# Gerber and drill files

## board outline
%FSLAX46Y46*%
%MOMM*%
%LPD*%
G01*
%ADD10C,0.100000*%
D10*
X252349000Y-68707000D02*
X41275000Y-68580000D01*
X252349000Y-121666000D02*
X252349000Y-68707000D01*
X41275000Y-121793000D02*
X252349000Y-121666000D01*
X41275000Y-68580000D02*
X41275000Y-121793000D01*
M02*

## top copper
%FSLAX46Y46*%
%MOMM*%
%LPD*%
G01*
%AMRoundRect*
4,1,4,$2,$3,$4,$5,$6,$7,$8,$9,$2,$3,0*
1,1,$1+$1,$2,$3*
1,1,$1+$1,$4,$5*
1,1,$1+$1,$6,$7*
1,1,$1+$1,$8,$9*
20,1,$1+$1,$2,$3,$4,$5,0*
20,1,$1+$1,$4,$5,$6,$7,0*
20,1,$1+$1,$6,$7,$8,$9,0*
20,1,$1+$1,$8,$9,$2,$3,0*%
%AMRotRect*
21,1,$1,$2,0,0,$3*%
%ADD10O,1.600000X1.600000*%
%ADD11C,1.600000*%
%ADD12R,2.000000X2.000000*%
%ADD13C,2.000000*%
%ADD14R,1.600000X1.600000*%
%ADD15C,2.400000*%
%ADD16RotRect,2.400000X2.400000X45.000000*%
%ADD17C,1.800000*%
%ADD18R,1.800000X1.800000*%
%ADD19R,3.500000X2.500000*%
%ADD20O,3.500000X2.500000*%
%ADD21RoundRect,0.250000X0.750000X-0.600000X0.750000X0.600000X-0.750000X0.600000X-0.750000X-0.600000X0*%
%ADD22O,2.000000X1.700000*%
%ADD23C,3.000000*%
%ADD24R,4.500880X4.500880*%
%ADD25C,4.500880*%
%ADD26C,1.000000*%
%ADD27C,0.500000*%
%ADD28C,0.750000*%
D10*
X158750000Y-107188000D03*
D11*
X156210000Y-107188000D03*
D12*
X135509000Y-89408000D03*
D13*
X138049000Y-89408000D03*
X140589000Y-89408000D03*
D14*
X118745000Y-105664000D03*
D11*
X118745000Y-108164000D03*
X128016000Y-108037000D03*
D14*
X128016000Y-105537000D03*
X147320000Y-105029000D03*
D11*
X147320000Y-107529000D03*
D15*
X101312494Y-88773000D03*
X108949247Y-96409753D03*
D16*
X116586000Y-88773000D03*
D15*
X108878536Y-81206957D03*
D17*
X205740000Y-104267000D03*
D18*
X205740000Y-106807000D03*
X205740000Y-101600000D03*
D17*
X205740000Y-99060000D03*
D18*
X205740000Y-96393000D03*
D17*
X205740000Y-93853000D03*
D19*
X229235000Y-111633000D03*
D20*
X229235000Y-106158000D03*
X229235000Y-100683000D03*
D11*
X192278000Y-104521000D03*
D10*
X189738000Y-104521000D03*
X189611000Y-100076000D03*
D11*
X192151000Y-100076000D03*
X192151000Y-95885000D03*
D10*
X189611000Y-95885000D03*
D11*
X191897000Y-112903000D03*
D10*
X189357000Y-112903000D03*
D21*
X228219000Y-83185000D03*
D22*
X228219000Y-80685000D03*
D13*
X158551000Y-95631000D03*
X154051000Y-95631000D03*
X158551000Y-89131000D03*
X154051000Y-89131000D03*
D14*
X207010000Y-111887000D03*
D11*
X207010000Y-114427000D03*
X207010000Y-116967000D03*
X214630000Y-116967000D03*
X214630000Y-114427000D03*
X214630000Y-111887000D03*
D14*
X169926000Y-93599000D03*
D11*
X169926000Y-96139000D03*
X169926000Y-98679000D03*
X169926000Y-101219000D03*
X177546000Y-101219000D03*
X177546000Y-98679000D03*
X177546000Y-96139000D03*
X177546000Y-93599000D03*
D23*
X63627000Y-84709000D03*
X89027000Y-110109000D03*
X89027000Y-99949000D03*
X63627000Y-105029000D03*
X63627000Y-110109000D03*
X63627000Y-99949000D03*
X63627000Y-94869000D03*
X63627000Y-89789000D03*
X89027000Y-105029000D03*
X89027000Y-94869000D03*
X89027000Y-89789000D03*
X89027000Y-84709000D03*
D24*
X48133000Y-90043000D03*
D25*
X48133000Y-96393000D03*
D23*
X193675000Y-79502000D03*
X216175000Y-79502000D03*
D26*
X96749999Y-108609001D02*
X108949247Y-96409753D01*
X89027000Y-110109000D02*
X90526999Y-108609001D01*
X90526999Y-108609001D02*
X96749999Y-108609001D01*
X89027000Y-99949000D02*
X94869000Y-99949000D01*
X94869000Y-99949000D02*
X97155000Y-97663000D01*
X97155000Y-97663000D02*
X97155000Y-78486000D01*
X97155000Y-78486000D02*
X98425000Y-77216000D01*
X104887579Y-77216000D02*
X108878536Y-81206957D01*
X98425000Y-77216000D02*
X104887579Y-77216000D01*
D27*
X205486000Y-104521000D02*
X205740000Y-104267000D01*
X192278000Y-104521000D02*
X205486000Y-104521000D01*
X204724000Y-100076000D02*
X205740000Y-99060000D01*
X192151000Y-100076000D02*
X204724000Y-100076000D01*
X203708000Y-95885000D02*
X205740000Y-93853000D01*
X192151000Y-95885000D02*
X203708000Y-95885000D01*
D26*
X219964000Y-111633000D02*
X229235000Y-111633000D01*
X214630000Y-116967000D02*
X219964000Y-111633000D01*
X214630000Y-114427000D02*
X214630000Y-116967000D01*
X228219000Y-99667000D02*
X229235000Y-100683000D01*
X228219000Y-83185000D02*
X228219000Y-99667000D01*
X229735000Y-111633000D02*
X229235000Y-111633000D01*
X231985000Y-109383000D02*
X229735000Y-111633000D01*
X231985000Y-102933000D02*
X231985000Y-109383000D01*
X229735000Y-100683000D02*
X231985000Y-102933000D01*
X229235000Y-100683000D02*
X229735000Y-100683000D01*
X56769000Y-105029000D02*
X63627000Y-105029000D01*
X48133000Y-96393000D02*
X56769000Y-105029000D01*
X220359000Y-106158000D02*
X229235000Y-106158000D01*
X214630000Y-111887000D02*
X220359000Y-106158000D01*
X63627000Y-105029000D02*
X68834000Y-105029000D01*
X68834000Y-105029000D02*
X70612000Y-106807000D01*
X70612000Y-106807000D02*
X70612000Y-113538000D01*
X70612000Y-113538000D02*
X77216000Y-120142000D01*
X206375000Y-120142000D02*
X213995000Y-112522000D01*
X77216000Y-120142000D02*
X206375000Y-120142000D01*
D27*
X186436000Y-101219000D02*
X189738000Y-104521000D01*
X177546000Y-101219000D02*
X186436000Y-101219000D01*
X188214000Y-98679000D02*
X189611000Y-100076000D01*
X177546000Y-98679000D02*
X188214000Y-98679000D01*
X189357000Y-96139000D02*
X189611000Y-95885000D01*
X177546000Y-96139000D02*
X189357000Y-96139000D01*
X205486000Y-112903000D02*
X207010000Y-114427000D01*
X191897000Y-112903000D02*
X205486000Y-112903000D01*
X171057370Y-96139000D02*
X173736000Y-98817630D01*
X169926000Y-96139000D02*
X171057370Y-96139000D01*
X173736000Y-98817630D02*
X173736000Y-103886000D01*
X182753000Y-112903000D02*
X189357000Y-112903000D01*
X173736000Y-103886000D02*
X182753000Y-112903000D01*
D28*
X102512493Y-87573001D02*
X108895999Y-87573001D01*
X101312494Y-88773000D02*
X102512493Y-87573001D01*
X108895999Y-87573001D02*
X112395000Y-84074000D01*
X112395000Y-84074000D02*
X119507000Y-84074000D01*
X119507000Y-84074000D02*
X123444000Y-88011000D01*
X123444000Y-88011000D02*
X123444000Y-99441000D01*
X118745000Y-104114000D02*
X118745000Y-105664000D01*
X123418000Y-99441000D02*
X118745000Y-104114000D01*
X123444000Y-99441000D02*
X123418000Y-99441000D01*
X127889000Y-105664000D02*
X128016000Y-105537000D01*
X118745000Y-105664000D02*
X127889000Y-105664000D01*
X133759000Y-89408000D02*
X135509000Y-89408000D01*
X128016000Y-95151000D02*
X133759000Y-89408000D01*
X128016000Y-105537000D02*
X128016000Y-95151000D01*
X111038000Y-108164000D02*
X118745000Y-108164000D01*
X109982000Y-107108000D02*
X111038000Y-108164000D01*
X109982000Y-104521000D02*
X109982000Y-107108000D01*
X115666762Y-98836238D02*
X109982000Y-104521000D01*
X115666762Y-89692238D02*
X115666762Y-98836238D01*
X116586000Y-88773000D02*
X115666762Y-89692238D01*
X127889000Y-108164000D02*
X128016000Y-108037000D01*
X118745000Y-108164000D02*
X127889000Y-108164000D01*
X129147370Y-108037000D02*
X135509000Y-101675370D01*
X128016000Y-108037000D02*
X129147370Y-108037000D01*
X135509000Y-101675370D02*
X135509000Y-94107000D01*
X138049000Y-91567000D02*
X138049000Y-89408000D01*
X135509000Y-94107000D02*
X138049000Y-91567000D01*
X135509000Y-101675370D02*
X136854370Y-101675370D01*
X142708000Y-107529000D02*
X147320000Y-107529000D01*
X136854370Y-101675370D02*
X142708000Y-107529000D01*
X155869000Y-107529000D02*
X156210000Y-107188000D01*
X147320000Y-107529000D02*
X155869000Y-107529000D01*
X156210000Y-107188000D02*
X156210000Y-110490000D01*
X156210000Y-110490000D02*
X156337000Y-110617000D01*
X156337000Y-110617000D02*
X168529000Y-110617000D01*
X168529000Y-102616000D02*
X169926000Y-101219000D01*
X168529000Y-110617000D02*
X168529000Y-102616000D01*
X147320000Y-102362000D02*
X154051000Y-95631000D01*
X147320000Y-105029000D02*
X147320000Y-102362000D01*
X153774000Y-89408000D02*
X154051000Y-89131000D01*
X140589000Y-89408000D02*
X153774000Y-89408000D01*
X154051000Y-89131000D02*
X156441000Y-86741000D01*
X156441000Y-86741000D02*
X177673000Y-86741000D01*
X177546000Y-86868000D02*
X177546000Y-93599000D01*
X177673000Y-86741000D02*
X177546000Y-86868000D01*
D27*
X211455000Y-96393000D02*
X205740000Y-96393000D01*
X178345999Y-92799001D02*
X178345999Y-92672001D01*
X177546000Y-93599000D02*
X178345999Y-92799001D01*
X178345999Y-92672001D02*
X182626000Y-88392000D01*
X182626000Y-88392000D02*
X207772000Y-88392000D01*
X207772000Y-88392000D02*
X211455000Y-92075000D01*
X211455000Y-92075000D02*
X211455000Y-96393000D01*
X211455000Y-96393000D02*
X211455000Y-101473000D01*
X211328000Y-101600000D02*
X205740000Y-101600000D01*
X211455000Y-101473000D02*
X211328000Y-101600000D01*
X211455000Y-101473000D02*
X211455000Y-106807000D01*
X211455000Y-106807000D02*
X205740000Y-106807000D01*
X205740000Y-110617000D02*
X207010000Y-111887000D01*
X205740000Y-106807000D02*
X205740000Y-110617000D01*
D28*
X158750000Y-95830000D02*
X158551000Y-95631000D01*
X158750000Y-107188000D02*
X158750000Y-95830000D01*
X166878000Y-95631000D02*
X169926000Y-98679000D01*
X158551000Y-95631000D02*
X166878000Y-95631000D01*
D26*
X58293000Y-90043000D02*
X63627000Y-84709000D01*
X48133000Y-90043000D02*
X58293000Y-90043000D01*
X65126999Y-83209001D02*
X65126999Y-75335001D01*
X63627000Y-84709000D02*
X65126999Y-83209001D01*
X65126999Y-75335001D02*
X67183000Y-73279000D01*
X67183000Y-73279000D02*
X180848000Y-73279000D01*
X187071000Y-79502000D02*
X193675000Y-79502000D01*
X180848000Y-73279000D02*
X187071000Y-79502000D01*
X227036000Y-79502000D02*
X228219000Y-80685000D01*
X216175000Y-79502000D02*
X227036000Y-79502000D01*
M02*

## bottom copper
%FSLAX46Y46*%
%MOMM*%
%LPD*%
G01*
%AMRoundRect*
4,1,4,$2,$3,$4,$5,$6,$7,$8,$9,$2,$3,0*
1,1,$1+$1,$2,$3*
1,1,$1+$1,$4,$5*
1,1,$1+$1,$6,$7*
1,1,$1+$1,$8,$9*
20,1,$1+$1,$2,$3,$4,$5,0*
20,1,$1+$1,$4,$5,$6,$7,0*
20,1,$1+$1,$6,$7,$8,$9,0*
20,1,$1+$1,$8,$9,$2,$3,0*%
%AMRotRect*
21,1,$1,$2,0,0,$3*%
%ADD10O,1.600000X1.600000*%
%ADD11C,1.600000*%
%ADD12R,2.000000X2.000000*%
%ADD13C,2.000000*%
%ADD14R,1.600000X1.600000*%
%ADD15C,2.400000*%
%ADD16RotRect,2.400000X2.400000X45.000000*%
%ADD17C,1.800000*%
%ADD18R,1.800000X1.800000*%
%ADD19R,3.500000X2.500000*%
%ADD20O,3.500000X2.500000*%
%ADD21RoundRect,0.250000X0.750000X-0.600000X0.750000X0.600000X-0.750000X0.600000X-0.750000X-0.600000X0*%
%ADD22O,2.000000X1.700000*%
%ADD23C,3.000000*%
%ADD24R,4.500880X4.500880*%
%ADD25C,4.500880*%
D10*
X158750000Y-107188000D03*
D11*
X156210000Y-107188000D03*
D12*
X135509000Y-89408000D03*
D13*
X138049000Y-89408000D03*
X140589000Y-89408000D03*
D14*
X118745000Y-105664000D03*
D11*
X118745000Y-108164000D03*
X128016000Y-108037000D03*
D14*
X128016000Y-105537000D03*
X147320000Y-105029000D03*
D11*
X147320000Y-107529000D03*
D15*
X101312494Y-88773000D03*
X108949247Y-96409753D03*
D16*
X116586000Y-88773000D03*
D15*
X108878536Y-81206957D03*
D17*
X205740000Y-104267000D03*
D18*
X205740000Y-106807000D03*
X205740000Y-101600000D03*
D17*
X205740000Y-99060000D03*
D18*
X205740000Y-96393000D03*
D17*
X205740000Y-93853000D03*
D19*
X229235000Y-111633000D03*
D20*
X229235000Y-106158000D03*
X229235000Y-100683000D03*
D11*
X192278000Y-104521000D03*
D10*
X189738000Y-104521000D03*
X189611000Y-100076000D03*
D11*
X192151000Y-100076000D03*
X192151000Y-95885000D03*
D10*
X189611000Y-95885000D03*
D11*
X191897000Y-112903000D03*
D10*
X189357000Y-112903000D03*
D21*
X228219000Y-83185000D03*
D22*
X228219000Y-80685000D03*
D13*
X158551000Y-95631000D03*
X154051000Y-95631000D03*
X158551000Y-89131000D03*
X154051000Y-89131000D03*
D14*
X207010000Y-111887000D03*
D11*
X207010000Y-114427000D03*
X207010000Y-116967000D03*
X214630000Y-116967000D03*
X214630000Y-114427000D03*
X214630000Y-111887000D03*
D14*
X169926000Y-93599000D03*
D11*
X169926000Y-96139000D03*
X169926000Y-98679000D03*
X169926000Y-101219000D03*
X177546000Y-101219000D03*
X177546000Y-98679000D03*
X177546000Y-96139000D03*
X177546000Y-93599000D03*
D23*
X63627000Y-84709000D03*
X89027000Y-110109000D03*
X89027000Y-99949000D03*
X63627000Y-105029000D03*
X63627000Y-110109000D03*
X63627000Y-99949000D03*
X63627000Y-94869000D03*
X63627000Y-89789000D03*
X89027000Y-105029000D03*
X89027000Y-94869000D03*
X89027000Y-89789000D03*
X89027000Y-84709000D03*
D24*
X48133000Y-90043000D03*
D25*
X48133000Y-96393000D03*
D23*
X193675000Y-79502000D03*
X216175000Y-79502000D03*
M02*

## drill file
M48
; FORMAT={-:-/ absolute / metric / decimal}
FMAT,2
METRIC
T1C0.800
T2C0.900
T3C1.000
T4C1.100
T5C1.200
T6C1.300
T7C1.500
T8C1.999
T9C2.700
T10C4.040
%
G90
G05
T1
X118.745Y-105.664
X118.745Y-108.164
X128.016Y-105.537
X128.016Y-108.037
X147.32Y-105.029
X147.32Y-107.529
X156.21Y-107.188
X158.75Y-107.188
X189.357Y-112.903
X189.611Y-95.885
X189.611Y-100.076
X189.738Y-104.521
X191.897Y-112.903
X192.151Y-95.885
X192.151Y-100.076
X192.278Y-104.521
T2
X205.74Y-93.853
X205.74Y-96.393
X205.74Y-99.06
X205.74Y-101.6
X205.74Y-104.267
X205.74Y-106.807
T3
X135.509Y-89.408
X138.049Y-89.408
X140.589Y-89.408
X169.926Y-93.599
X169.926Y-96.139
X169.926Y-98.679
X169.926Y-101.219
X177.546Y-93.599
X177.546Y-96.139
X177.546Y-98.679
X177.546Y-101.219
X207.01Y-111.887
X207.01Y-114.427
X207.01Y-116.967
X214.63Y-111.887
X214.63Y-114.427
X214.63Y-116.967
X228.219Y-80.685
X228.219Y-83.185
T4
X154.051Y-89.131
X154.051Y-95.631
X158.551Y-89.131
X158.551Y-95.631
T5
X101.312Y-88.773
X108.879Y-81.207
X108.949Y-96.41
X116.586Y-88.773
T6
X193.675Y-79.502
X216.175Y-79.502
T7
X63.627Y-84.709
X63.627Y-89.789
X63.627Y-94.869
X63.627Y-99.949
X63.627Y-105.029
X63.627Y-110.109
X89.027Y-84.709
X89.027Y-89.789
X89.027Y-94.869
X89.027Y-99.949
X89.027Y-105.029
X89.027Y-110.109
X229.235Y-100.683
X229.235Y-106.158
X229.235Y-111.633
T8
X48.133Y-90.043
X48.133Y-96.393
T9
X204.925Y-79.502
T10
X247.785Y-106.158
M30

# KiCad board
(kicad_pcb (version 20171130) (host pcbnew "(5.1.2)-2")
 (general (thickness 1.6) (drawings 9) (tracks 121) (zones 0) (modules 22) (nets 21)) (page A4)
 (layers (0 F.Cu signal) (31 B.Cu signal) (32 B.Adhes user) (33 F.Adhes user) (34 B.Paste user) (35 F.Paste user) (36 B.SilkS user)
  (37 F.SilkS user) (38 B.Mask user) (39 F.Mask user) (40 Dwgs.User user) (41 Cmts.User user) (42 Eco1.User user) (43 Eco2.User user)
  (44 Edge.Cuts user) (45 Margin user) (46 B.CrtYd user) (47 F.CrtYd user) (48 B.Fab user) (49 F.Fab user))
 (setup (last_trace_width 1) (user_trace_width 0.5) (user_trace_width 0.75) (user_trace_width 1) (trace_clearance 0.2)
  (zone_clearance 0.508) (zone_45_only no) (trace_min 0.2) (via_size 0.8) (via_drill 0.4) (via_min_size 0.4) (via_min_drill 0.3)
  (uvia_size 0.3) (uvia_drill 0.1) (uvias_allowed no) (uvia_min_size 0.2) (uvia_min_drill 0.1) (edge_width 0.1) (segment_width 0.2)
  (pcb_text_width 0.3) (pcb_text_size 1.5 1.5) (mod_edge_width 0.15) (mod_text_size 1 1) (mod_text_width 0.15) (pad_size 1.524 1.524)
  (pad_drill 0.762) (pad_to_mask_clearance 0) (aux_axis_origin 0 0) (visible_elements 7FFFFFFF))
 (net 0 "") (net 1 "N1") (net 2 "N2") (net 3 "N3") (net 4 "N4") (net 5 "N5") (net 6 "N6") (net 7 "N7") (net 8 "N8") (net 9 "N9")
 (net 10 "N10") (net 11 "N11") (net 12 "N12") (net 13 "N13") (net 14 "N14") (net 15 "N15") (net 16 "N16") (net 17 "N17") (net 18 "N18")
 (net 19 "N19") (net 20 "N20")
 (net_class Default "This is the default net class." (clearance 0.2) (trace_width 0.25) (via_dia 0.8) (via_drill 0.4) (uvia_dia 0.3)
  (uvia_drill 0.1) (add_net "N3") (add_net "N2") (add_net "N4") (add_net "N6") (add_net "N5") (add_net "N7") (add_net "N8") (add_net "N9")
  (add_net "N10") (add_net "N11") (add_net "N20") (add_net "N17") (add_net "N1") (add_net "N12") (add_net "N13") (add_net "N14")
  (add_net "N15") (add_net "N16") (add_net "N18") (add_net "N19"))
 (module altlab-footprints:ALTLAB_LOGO (layer F.Cu) (at 136.271 78.867)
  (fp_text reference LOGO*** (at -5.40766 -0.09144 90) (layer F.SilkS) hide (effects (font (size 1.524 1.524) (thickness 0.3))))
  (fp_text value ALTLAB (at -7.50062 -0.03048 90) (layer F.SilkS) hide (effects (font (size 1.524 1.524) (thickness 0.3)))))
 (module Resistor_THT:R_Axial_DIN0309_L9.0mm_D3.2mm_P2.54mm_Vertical (layer F.Cu) (at 156.21 107.188)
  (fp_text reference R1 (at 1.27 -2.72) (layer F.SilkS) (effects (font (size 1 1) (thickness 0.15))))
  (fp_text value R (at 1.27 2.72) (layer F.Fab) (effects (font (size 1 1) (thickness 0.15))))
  (pad 2 thru_hole oval (at 2.54 0) (size 1.6 1.6) (drill 0.8) (layers *.Cu *.Mask) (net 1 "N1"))
  (pad 1 thru_hole circle (at 0 0) (size 1.6 1.6) (drill 0.8) (layers *.Cu *.Mask) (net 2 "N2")))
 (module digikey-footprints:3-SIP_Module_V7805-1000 (layer F.Cu) (at 135.509 89.408)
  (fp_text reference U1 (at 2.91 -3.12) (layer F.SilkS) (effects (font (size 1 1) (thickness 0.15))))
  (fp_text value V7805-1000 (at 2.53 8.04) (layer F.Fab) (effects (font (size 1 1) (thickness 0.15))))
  (pad 1 thru_hole rect (at 0 0) (size 2 2) (drill 1) (layers *.Cu *.Mask) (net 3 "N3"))
  (pad 2 thru_hole circle (at 2.54 0) (size 2 2) (drill 1) (layers *.Cu *.Mask) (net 2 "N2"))
  (pad 3 thru_hole circle (at 5.08 0) (size 2 2) (drill 1) (layers *.Cu *.Mask) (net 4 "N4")))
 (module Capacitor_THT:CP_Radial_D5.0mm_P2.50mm (layer F.Cu) (at 118.745 105.664 270)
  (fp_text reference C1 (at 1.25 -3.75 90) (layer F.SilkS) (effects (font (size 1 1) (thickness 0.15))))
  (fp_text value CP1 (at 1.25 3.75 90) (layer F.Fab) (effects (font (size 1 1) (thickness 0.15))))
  (pad 1 thru_hole rect (at 0 0 270) (size 1.6 1.6) (drill 0.8) (layers *.Cu *.Mask) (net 3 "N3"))
  (pad 2 thru_hole circle (at 2.5 0 270) (size 1.6 1.6) (drill 0.8) (layers *.Cu *.Mask) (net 2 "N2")))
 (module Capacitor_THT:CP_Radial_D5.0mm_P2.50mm (layer F.Cu) (at 128.016 105.537 270)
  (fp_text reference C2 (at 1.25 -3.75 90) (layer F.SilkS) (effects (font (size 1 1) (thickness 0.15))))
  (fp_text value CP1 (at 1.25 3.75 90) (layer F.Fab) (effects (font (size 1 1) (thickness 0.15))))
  (pad 2 thru_hole circle (at 2.5 0 270) (size 1.6 1.6) (drill 0.8) (layers *.Cu *.Mask) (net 2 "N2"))
  (pad 1 thru_hole rect (at 0 0 270) (size 1.6 1.6) (drill 0.8) (layers *.Cu *.Mask) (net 3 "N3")))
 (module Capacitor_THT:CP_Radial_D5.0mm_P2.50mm (layer F.Cu) (at 147.32 105.029 270)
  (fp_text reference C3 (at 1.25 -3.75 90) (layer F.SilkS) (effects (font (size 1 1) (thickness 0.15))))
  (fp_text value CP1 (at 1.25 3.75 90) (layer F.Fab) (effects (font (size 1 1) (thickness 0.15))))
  (pad 1 thru_hole rect (at 0 0 270) (size 1.6 1.6) (drill 0.8) (layers *.Cu *.Mask) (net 4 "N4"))
  (pad 2 thru_hole circle (at 2.5 0 270) (size 1.6 1.6) (drill 0.8) (layers *.Cu *.Mask) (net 2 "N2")))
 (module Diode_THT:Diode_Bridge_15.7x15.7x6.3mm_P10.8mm (layer F.Cu) (at 116.586 88.773 225)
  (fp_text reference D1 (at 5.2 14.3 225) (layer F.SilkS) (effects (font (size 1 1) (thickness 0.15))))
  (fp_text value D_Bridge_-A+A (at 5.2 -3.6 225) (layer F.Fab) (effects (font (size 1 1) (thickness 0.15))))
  (pad 3 thru_hole circle (at 10.8 10.8 45) (size 2.4 2.4) (drill 1.2) (layers *.Cu *.Mask) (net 3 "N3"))
  (pad 4 thru_hole circle (at 10.8 0 45) (size 2.4 2.4) (drill 1.2) (layers *.Cu *.Mask) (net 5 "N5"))
  (pad 1 thru_hole rect (at 0 0 45) (size 2.4 2.4) (drill 1.2) (layers *.Cu *.Mask) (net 2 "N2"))
  (pad 2 thru_hole circle (at 0.1 10.8 45) (size 2.4 2.4) (drill 1.2) (layers *.Cu *.Mask) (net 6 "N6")))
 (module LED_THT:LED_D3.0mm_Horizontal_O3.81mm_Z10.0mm (layer F.Cu) (at 205.74 106.807 90)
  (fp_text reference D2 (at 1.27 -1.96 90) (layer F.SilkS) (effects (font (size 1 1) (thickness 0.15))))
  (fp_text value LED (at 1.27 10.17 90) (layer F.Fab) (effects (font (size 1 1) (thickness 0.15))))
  (pad 2 thru_hole circle (at 2.54 0 90) (size 1.8 1.8) (drill 0.9) (layers *.Cu *.Mask) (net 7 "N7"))
  (pad 1 thru_hole rect (at 0 0 90) (size 1.8 1.8) (drill 0.9) (layers *.Cu *.Mask) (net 4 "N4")))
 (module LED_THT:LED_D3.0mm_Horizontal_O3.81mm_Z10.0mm (layer F.Cu) (at 205.74 101.6 90)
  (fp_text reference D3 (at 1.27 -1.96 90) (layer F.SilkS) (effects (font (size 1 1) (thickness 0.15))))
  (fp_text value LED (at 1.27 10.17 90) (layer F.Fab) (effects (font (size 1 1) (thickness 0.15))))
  (pad 1 thru_hole rect (at 0 0 90) (size 1.8 1.8) (drill 0.9) (layers *.Cu *.Mask) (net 4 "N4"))
  (pad 2 thru_hole circle (at 2.54 0 90) (size 1.8 1.8) (drill 0.9) (layers *.Cu *.Mask) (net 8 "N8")))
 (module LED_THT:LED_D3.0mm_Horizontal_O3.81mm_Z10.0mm (layer F.Cu) (at 205.74 96.393 90)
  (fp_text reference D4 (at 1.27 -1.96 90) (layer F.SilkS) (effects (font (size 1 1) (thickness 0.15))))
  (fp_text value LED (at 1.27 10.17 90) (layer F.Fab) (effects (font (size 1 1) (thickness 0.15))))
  (pad 1 thru_hole rect (at 0 0 90) (size 1.8 1.8) (drill 0.9) (layers *.Cu *.Mask) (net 4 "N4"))
  (pad 2 thru_hole circle (at 2.54 0 90) (size 1.8 1.8) (drill 0.9) (layers *.Cu *.Mask) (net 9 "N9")))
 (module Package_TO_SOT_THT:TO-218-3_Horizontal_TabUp (layer F.Cu) (at 229.235 111.633 90)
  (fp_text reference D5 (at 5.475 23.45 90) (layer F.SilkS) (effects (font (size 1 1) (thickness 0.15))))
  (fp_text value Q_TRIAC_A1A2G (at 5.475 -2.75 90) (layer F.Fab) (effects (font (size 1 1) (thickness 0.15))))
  (pad "" np_thru_hole oval (at 5.475 18.55 90) (size 4.04 4.04) (drill 4.04) (layers *.Cu *.Mask))
  (pad 1 thru_hole rect (at 0 0 90) (size 2.5 3.5) (drill 1.5) (layers *.Cu *.Mask) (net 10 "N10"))
  (pad 2 thru_hole oval (at 5.475 0 90) (size 2.5 3.5) (drill 1.5) (layers *.Cu *.Mask) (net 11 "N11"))
  (pad 3 thru_hole oval (at 10.95 0 90) (size 2.5 3.5) (drill 1.5) (layers *.Cu *.Mask) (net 10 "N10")))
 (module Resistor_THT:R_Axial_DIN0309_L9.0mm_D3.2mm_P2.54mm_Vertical (layer F.Cu) (at 192.278 104.521 180)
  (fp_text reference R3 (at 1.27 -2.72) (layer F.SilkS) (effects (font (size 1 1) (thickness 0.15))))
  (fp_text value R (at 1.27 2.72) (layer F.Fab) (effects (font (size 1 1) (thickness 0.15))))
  (pad 1 thru_hole circle (at 0 0 180) (size 1.6 1.6) (drill 0.8) (layers *.Cu *.Mask) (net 7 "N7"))
  (pad 2 thru_hole oval (at 2.54 0 180) (size 1.6 1.6) (drill 0.8) (layers *.Cu *.Mask) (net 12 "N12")))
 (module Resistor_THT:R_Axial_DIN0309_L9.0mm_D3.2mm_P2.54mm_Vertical (layer F.Cu) (at 192.151 100.076 180)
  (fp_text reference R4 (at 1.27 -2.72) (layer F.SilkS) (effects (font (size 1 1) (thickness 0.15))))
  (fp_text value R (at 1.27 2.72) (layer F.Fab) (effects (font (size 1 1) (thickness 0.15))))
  (pad 2 thru_hole oval (at 2.54 0 180) (size 1.6 1.6) (drill 0.8) (layers *.Cu *.Mask) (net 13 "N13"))
  (pad 1 thru_hole circle (at 0 0 180) (size 1.6 1.6) (drill 0.8) (layers *.Cu *.Mask) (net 8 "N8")))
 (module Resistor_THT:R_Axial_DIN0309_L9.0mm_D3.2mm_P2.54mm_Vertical (layer F.Cu) (at 192.151 95.885 180)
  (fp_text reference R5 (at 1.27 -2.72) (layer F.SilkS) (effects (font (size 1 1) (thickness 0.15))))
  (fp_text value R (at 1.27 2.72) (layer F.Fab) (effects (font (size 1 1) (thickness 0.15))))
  (pad 1 thru_hole circle (at 0 0 180) (size 1.6 1.6) (drill 0.8) (layers *.Cu *.Mask) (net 9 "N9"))
  (pad 2 thru_hole oval (at 2.54 0 180) (size 1.6 1.6) (drill 0.8) (layers *.Cu *.Mask) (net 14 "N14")))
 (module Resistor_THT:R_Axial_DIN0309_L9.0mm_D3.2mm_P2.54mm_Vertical (layer F.Cu) (at 191.897 112.903 180)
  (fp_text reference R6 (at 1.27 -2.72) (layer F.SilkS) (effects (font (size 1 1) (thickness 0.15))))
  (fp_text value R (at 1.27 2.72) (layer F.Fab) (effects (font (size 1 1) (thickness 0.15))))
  (pad 1 thru_hole circle (at 0 0 180) (size 1.6 1.6) (drill 0.8) (layers *.Cu *.Mask) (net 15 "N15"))
  (pad 2 thru_hole oval (at 2.54 0 180) (size 1.6 1.6) (drill 0.8) (layers *.Cu *.Mask) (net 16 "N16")))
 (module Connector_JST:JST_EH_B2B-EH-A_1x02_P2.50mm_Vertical (layer F.Cu) (at 228.219 83.185 90)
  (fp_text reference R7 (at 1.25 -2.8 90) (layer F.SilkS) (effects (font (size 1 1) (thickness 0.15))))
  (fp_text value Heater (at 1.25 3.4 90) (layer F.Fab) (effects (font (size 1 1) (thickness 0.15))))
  (pad 1 thru_hole roundrect (at 0 0 90) (size 1.7 2) (drill 1) (layers *.Cu *.Mask) (roundrect_rratio 0.147059) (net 10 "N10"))
  (pad 2 thru_hole oval (at 2.5 0 90) (size 1.7 2) (drill 1) (layers *.Cu *.Mask) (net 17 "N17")))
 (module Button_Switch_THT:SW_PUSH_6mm (layer F.Cu) (at 154.051 95.631 90)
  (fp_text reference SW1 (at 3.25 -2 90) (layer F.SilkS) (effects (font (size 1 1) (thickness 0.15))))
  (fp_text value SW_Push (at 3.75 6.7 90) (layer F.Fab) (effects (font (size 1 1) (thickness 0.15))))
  (pad 2 thru_hole circle (at 0 4.5 180) (size 2 2) (drill 1.1) (layers *.Cu *.Mask) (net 1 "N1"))
  (pad 1 thru_hole circle (at 0 0 180) (size 2 2) (drill 1.1) (layers *.Cu *.Mask) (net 4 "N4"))
  (pad 2 thru_hole circle (at 6.5 4.5 180) (size 2 2) (drill 1.1) (layers *.Cu *.Mask) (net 1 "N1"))
  (pad 1 thru_hole circle (at 6.5 0 180) (size 2 2) (drill 1.1) (layers *.Cu *.Mask) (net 4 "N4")))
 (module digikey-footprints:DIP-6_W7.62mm (layer F.Cu) (at 207.01 111.887)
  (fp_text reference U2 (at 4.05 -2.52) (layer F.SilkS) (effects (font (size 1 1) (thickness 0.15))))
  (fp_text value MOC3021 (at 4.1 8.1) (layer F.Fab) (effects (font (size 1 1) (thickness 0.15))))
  (pad 1 thru_hole rect (at 0 0) (size 1.6 1.6) (drill 1) (layers *.Cu *.Mask) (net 4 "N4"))
  (pad 2 thru_hole circle (at 0 2.54) (size 1.6 1.6) (drill 1) (layers *.Cu *.Mask) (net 15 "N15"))
  (pad 3 thru_hole circle (at 0 5.08) (size 1.6 1.6) (drill 1) (layers *.Cu *.Mask) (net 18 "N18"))
  (pad 4 thru_hole circle (at 7.62 5.08) (size 1.6 1.6) (drill 1) (layers *.Cu *.Mask) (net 10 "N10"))
  (pad 5 thru_hole circle (at 7.62 2.54) (size 1.6 1.6) (drill 1) (layers *.Cu *.Mask) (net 10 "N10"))
  (pad 6 thru_hole circle (at 7.62 0) (size 1.6 1.6) (drill 1) (layers *.Cu *.Mask) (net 11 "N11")))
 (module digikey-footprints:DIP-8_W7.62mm (layer F.Cu) (at 169.926 93.599)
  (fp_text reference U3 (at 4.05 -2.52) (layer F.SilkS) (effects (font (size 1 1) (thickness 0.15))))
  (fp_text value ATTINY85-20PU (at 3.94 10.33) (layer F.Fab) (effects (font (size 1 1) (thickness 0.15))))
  (pad 1 thru_hole rect (at 0 0) (size 1.6 1.6) (drill 1) (layers *.Cu *.Mask) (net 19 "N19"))
  (pad 2 thru_hole circle (at 0 2.54) (size 1.6 1.6) (drill 1) (layers *.Cu *.Mask) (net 16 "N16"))
  (pad 3 thru_hole circle (at 0 5.08) (size 1.6 1.6) (drill 1) (layers *.Cu *.Mask) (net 1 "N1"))
  (pad 4 thru_hole circle (at 0 7.62) (size 1.6 1.6) (drill 1) (layers *.Cu *.Mask) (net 2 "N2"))
  (pad 5 thru_hole circle (at 7.62 7.62) (size 1.6 1.6) (drill 1) (layers *.Cu *.Mask) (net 12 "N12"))
  (pad 6 thru_hole circle (at 7.62 5.08) (size 1.6 1.6) (drill 1) (layers *.Cu *.Mask) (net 13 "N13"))
  (pad 7 thru_hole circle (at 7.62 2.54) (size 1.6 1.6) (drill 1) (layers *.Cu *.Mask) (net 14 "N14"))
  (pad 8 thru_hole circle (at 7.62 0) (size 1.6 1.6) (drill 1) (layers *.Cu *.Mask) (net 4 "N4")))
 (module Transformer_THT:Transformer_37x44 (layer F.Cu) (at 63.627 105.029 90)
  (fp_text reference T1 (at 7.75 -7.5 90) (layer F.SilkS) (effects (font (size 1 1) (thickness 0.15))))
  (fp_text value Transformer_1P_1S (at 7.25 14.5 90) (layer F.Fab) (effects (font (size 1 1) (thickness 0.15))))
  (pad 2 thru_hole circle (at 20.32 0 90) (size 3 3) (drill 1.5) (layers *.Cu *.Mask) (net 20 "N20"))
  (pad 4 thru_hole circle (at -5.08 25.4 90) (size 3 3) (drill 1.5) (layers *.Cu *.Mask) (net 5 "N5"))
  (pad 3 thru_hole circle (at 5.08 25.4 90) (size 3 3) (drill 1.5) (layers *.Cu *.Mask) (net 6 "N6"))
  (pad 1 thru_hole circle (at 0 0 90) (size 3 3) (drill 1.5) (layers *.Cu *.Mask) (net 11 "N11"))
  (pad "" thru_hole circle (at -5.08 0 90) (size 3 3) (drill 1.5) (layers *.Cu *.Mask))
  (pad "" thru_hole circle (at 5.08 0 90) (size 3 3) (drill 1.5) (layers *.Cu *.Mask))
  (pad "" thru_hole circle (at 10.16 0 90) (size 3 3) (drill 1.5) (layers *.Cu *.Mask))
  (pad "" thru_hole circle (at 15.24 0 90) (size 3 3) (drill 1.5) (layers *.Cu *.Mask))
  (pad "" thru_hole circle (at 0 25.4 90) (size 3 3) (drill 1.5) (layers *.Cu *.Mask))
  (pad "" thru_hole circle (at 10.16 25.4 90) (size 3 3) (drill 1.5) (layers *.Cu *.Mask))
  (pad "" thru_hole circle (at 15.24 25.4 90) (size 3 3) (drill 1.5) (layers *.Cu *.Mask))
  (pad "" thru_hole circle (at 20.32 25.4 90) (size 3 3) (drill 1.5) (layers *.Cu *.Mask)))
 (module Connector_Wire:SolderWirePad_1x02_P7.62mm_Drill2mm (layer F.Cu) (at 48.133 90.043 270)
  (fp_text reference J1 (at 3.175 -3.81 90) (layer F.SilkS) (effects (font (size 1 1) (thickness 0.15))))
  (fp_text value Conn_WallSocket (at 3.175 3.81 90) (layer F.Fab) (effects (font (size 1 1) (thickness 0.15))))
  (pad 1 thru_hole rect (at 0 0 270) (size 4.50088 4.50088) (drill 1.99898) (layers *.Cu *.Mask) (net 20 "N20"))
  (pad 2 thru_hole circle (at 6.35 0 270) (size 4.50088 4.50088) (drill 1.99898) (layers *.Cu *.Mask) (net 11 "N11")))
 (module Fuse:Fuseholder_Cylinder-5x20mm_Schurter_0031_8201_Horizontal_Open (layer F.Cu) (at 193.675 79.502)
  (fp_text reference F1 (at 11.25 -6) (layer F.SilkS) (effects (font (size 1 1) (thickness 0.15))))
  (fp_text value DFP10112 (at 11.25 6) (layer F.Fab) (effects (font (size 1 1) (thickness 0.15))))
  (pad 1 thru_hole circle (at 0 0) (size 3 3) (drill 1.3) (layers *.Cu *.Mask) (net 20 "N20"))
  (pad 2 thru_hole circle (at 22.5 0) (size 3 3) (drill 1.3) (layers *.Cu *.Mask) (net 17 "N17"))
  (pad "" np_thru_hole circle (at 11.25 0) (size 2.7 2.7) (drill 2.7) (layers *.Cu *.Mask)))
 (gr_line (start 252.349 68.707) (end 41.275 68.58) (layer Edge.Cuts) (width 0.1))
 (gr_line (start 252.349 121.666) (end 252.349 68.707) (layer Edge.Cuts) (width 0.1))
 (gr_line (start 41.275 121.793) (end 252.349 121.666) (layer Edge.Cuts) (width 0.1))
 (gr_line (start 41.275 68.58) (end 41.275 121.793) (layer Edge.Cuts) (width 0.1))
 (segment (start 96.749999 108.609001) (end 108.949247 96.409753) (width 1) (layer F.Cu) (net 5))
 (segment (start 89.027 110.109) (end 90.526999 108.609001) (width 1) (layer F.Cu) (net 5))
 (segment (start 90.526999 108.609001) (end 96.749999 108.609001) (width 1) (layer F.Cu) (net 5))
 (segment (start 89.027 99.949) (end 94.869 99.949) (width 1) (layer F.Cu) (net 6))
 (segment (start 94.869 99.949) (end 97.155 97.663) (width 1) (layer F.Cu) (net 6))
 (segment (start 97.155 97.663) (end 97.155 78.486) (width 1) (layer F.Cu) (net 6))
 (segment (start 97.155 78.486) (end 98.425 77.216) (width 1) (layer F.Cu) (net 6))
 (segment (start 104.887579 77.216) (end 108.878536 81.206957) (width 1) (layer F.Cu) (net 6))
 (segment (start 98.425 77.216) (end 104.887579 77.216) (width 1) (layer F.Cu) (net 6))
 (segment (start 205.486 104.521) (end 205.74 104.267) (width 0.5) (layer F.Cu) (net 7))
 (segment (start 192.278 104.521) (end 205.486 104.521) (width 0.5) (layer F.Cu) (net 7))
 (segment (start 204.724 100.076) (end 205.74 99.06) (width 0.5) (layer F.Cu) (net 8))
 (segment (start 192.151 100.076) (end 204.724 100.076) (width 0.5) (layer F.Cu) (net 8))
 (segment (start 203.708 95.885) (end 205.74 93.853) (width 0.5) (layer F.Cu) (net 9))
 (segment (start 192.151 95.885) (end 203.708 95.885) (width 0.5) (layer F.Cu) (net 9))
 (segment (start 219.964 111.633) (end 229.235 111.633) (width 1) (layer F.Cu) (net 10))
 (segment (start 214.63 116.967) (end 219.964 111.633) (width 1) (layer F.Cu) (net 10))
 (segment (start 214.63 114.427) (end 214.63 116.967) (width 1) (layer F.Cu) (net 10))
 (segment (start 228.219 99.667) (end 229.235 100.683) (width 1) (layer F.Cu) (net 10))
 (segment (start 228.219 83.185) (end 228.219 99.667) (width 1) (layer F.Cu) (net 10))
 (segment (start 229.735 111.633) (end 229.235 111.633) (width 1) (layer F.Cu) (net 10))
 (segment (start 231.985 109.383) (end 229.735 111.633) (width 1) (layer F.Cu) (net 10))
 (segment (start 231.985 102.933) (end 231.985 109.383) (width 1) (layer F.Cu) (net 10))
 (segment (start 229.735 100.683) (end 231.985 102.933) (width 1) (layer F.Cu) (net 10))
 (segment (start 229.235 100.683) (end 229.735 100.683) (width 1) (layer F.Cu) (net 10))
 (segment (start 56.769 105.029) (end 63.627 105.029) (width 1) (layer F.Cu) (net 11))
 (segment (start 48.133 96.393) (end 56.769 105.029) (width 1) (layer F.Cu) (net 11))
 (segment (start 220.359 106.158) (end 229.235 106.158) (width 1) (layer F.Cu) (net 11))
 (segment (start 214.63 111.887) (end 220.359 106.158) (width 1) (layer F.Cu) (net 11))
 (segment (start 63.627 105.029) (end 68.834 105.029) (width 1) (layer F.Cu) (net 11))
 (segment (start 68.834 105.029) (end 70.612 106.807) (width 1) (layer F.Cu) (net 11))
 (segment (start 70.612 106.807) (end 70.612 113.538) (width 1) (layer F.Cu) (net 11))
 (segment (start 70.612 113.538) (end 77.216 120.142) (width 1) (layer F.Cu) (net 11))
 (segment (start 206.375 120.142) (end 213.995 112.522) (width 1) (layer F.Cu) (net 11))
 (segment (start 77.216 120.142) (end 206.375 120.142) (width 1) (layer F.Cu) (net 11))
 (segment (start 186.436 101.219) (end 189.738 104.521) (width 0.5) (layer F.Cu) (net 12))
 (segment (start 177.546 101.219) (end 186.436 101.219) (width 0.5) (layer F.Cu) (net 12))
 (segment (start 188.214 98.679) (end 189.611 100.076) (width 0.5) (layer F.Cu) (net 13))
 (segment (start 177.546 98.679) (end 188.214 98.679) (width 0.5) (layer F.Cu) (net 13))
 (segment (start 189.357 96.139) (end 189.611 95.885) (width 0.5) (layer F.Cu) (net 14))
 (segment (start 177.546 96.139) (end 189.357 96.139) (width 0.5) (layer F.Cu) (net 14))
 (segment (start 205.486 112.903) (end 207.01 114.427) (width 0.5) (layer F.Cu) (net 15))
 (segment (start 191.897 112.903) (end 205.486 112.903) (width 0.5) (layer F.Cu) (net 15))
 (segment (start 171.05737 96.139) (end 173.736 98.81763) (width 0.5) (layer F.Cu) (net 16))
 (segment (start 169.926 96.139) (end 171.05737 96.139) (width 0.5) (layer F.Cu) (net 16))
 (segment (start 173.736 98.81763) (end 173.736 103.886) (width 0.5) (layer F.Cu) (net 16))
 (segment (start 182.753 112.903) (end 189.357 112.903) (width 0.5) (layer F.Cu) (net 16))
 (segment (start 173.736 103.886) (end 182.753 112.903) (width 0.5) (layer F.Cu) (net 16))
 (segment (start 102.512493 87.573001) (end 108.895999 87.573001) (width 0.75) (layer F.Cu) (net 3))
 (segment (start 101.312494 88.773) (end 102.512493 87.573001) (width 0.75) (layer F.Cu) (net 3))
 (segment (start 108.895999 87.573001) (end 112.395 84.074) (width 0.75) (layer F.Cu) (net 3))
 (segment (start 112.395 84.074) (end 119.507 84.074) (width 0.75) (layer F.Cu) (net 3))
 (segment (start 119.507 84.074) (end 123.444 88.011) (width 0.75) (layer F.Cu) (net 3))
 (segment (start 123.444 88.011) (end 123.444 99.441) (width 0.75) (layer F.Cu) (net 3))
 (segment (start 118.745 104.114) (end 118.745 105.664) (width 0.75) (layer F.Cu) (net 3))
 (segment (start 123.418 99.441) (end 118.745 104.114) (width 0.75) (layer F.Cu) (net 3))
 (segment (start 123.444 99.441) (end 123.418 99.441) (width 0.75) (layer F.Cu) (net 3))
 (segment (start 127.889 105.664) (end 128.016 105.537) (width 0.75) (layer F.Cu) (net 3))
 (segment (start 118.745 105.664) (end 127.889 105.664) (width 0.75) (layer F.Cu) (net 3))
 (segment (start 133.759 89.408) (end 135.509 89.408) (width 0.75) (layer F.Cu) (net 3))
 (segment (start 128.016 95.151) (end 133.759 89.408) (width 0.75) (layer F.Cu) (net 3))
 (segment (start 128.016 105.537) (end 128.016 95.151) (width 0.75) (layer F.Cu) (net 3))
 (segment (start 111.038 108.164) (end 118.745 108.164) (width 0.75) (layer F.Cu) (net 2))
 (segment (start 109.982 107.108) (end 111.038 108.164) (width 0.75) (layer F.Cu) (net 2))
 (segment (start 109.982 104.521) (end 109.982 107.108) (width 0.75) (layer F.Cu) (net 2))
 (segment (start 115.666762 98.836238) (end 109.982 104.521) (width 0.75) (layer F.Cu) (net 2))
 (segment (start 115.666762 89.692238) (end 115.666762 98.836238) (width 0.75) (layer F.Cu) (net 2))
 (segment (start 116.586 88.773) (end 115.666762 89.692238) (width 0.75) (layer F.Cu) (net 2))
 (segment (start 127.889 108.164) (end 128.016 108.037) (width 0.75) (layer F.Cu) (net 2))
 (segment (start 118.745 108.164) (end 127.889 108.164) (width 0.75) (layer F.Cu) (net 2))
 (segment (start 129.14737 108.037) (end 135.509 101.67537) (width 0.75) (layer F.Cu) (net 2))
 (segment (start 128.016 108.037) (end 129.14737 108.037) (width 0.75) (layer F.Cu) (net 2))
 (segment (start 135.509 101.67537) (end 135.509 94.107) (width 0.75) (layer F.Cu) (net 2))
 (segment (start 138.049 91.567) (end 138.049 89.408) (width 0.75) (layer F.Cu) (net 2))
 (segment (start 135.509 94.107) (end 138.049 91.567) (width 0.75) (layer F.Cu) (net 2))
 (segment (start 135.509 101.67537) (end 136.85437 101.67537) (width 0.75) (layer F.Cu) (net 2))
 (segment (start 142.708 107.529) (end 147.32 107.529) (width 0.75) (layer F.Cu) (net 2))
 (segment (start 136.85437 101.67537) (end 142.708 107.529) (width 0.75) (layer F.Cu) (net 2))
 (segment (start 155.869 107.529) (end 156.21 107.188) (width 0.75) (layer F.Cu) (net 2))
 (segment (start 147.32 107.529) (end 155.869 107.529) (width 0.75) (layer F.Cu) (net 2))
 (segment (start 156.21 107.188) (end 156.21 110.49) (width 0.75) (layer F.Cu) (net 2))
 (segment (start 156.21 110.49) (end 156.337 110.617) (width 0.75) (layer F.Cu) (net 2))
 (segment (start 156.337 110.617) (end 168.529 110.617) (width 0.75) (layer F.Cu) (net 2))
 (segment (start 168.529 102.616) (end 169.926 101.219) (width 0.75) (layer F.Cu) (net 2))
 (segment (start 168.529 110.617) (end 168.529 102.616) (width 0.75) (layer F.Cu) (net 2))
 (segment (start 147.32 102.362) (end 154.051 95.631) (width 0.75) (layer F.Cu) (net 4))
 (segment (start 147.32 105.029) (end 147.32 102.362) (width 0.75) (layer F.Cu) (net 4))
 (segment (start 153.774 89.408) (end 154.051 89.131) (width 0.75) (layer F.Cu) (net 4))
 (segment (start 140.589 89.408) (end 153.774 89.408) (width 0.75) (layer F.Cu) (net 4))
 (segment (start 154.051 89.131) (end 156.441 86.741) (width 0.75) (layer F.Cu) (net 4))
 (segment (start 156.441 86.741) (end 177.673 86.741) (width 0.75) (layer F.Cu) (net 4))
 (segment (start 177.546 86.868) (end 177.546 93.599) (width 0.75) (layer F.Cu) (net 4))
 (segment (start 177.673 86.741) (end 177.546 86.868) (width 0.75) (layer F.Cu) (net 4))
 (segment (start 211.455 96.393) (end 205.74 96.393) (width 0.5) (layer F.Cu) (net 4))
 (segment (start 178.345999 92.799001) (end 178.345999 92.672001) (width 0.5) (layer F.Cu) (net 4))
 (segment (start 177.546 93.599) (end 178.345999 92.799001) (width 0.5) (layer F.Cu) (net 4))
 (segment (start 178.345999 92.672001) (end 182.626 88.392) (width 0.5) (layer F.Cu) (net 4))
 (segment (start 182.626 88.392) (end 207.772 88.392) (width 0.5) (layer F.Cu) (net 4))
 (segment (start 207.772 88.392) (end 211.455 92.075) (width 0.5) (layer F.Cu) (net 4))
 (segment (start 211.455 92.075) (end 211.455 96.393) (width 0.5) (layer F.Cu) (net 4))
 (segment (start 211.455 96.393) (end 211.455 101.473) (width 0.5) (layer F.Cu) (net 4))
 (segment (start 211.328 101.6) (end 205.74 101.6) (width 0.5) (layer F.Cu) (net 4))
 (segment (start 211.455 101.473) (end 211.328 101.6) (width 0.5) (layer F.Cu) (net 4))
 (segment (start 211.455 101.473) (end 211.455 106.807) (width 0.5) (layer F.Cu) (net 4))
 (segment (start 211.455 106.807) (end 205.74 106.807) (width 0.5) (layer F.Cu) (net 4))
 (segment (start 205.74 110.617) (end 207.01 111.887) (width 0.5) (layer F.Cu) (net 4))
 (segment (start 205.74 106.807) (end 205.74 110.617) (width 0.5) (layer F.Cu) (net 4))
 (segment (start 158.75 95.83) (end 158.551 95.631) (width 0.75) (layer F.Cu) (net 1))
 (segment (start 158.75 107.188) (end 158.75 95.83) (width 0.75) (layer F.Cu) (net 1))
 (segment (start 166.878 95.631) (end 169.926 98.679) (width 0.75) (layer F.Cu) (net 1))
 (segment (start 158.551 95.631) (end 166.878 95.631) (width 0.75) (layer F.Cu) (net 1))
 (segment (start 58.293 90.043) (end 63.627 84.709) (width 1) (layer F.Cu) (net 20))
 (segment (start 48.133 90.043) (end 58.293 90.043) (width 1) (layer F.Cu) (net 20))
 (segment (start 65.126999 83.209001) (end 65.126999 75.335001) (width 1) (layer F.Cu) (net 20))
 (segment (start 63.627 84.709) (end 65.126999 83.209001) (width 1) (layer F.Cu) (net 20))
 (segment (start 65.126999 75.335001) (end 67.183 73.279) (width 1) (layer F.Cu) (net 20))
 (segment (start 67.183 73.279) (end 180.848 73.279) (width 1) (layer F.Cu) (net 20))
 (segment (start 187.071 79.502) (end 193.675 79.502) (width 1) (layer F.Cu) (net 20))
 (segment (start 180.848 73.279) (end 187.071 79.502) (width 1) (layer F.Cu) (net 20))
 (segment (start 227.036 79.502) (end 228.219 80.685) (width 1) (layer F.Cu) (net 17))
 (segment (start 216.175 79.502) (end 227.036 79.502) (width 1) (layer F.Cu) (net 17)))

